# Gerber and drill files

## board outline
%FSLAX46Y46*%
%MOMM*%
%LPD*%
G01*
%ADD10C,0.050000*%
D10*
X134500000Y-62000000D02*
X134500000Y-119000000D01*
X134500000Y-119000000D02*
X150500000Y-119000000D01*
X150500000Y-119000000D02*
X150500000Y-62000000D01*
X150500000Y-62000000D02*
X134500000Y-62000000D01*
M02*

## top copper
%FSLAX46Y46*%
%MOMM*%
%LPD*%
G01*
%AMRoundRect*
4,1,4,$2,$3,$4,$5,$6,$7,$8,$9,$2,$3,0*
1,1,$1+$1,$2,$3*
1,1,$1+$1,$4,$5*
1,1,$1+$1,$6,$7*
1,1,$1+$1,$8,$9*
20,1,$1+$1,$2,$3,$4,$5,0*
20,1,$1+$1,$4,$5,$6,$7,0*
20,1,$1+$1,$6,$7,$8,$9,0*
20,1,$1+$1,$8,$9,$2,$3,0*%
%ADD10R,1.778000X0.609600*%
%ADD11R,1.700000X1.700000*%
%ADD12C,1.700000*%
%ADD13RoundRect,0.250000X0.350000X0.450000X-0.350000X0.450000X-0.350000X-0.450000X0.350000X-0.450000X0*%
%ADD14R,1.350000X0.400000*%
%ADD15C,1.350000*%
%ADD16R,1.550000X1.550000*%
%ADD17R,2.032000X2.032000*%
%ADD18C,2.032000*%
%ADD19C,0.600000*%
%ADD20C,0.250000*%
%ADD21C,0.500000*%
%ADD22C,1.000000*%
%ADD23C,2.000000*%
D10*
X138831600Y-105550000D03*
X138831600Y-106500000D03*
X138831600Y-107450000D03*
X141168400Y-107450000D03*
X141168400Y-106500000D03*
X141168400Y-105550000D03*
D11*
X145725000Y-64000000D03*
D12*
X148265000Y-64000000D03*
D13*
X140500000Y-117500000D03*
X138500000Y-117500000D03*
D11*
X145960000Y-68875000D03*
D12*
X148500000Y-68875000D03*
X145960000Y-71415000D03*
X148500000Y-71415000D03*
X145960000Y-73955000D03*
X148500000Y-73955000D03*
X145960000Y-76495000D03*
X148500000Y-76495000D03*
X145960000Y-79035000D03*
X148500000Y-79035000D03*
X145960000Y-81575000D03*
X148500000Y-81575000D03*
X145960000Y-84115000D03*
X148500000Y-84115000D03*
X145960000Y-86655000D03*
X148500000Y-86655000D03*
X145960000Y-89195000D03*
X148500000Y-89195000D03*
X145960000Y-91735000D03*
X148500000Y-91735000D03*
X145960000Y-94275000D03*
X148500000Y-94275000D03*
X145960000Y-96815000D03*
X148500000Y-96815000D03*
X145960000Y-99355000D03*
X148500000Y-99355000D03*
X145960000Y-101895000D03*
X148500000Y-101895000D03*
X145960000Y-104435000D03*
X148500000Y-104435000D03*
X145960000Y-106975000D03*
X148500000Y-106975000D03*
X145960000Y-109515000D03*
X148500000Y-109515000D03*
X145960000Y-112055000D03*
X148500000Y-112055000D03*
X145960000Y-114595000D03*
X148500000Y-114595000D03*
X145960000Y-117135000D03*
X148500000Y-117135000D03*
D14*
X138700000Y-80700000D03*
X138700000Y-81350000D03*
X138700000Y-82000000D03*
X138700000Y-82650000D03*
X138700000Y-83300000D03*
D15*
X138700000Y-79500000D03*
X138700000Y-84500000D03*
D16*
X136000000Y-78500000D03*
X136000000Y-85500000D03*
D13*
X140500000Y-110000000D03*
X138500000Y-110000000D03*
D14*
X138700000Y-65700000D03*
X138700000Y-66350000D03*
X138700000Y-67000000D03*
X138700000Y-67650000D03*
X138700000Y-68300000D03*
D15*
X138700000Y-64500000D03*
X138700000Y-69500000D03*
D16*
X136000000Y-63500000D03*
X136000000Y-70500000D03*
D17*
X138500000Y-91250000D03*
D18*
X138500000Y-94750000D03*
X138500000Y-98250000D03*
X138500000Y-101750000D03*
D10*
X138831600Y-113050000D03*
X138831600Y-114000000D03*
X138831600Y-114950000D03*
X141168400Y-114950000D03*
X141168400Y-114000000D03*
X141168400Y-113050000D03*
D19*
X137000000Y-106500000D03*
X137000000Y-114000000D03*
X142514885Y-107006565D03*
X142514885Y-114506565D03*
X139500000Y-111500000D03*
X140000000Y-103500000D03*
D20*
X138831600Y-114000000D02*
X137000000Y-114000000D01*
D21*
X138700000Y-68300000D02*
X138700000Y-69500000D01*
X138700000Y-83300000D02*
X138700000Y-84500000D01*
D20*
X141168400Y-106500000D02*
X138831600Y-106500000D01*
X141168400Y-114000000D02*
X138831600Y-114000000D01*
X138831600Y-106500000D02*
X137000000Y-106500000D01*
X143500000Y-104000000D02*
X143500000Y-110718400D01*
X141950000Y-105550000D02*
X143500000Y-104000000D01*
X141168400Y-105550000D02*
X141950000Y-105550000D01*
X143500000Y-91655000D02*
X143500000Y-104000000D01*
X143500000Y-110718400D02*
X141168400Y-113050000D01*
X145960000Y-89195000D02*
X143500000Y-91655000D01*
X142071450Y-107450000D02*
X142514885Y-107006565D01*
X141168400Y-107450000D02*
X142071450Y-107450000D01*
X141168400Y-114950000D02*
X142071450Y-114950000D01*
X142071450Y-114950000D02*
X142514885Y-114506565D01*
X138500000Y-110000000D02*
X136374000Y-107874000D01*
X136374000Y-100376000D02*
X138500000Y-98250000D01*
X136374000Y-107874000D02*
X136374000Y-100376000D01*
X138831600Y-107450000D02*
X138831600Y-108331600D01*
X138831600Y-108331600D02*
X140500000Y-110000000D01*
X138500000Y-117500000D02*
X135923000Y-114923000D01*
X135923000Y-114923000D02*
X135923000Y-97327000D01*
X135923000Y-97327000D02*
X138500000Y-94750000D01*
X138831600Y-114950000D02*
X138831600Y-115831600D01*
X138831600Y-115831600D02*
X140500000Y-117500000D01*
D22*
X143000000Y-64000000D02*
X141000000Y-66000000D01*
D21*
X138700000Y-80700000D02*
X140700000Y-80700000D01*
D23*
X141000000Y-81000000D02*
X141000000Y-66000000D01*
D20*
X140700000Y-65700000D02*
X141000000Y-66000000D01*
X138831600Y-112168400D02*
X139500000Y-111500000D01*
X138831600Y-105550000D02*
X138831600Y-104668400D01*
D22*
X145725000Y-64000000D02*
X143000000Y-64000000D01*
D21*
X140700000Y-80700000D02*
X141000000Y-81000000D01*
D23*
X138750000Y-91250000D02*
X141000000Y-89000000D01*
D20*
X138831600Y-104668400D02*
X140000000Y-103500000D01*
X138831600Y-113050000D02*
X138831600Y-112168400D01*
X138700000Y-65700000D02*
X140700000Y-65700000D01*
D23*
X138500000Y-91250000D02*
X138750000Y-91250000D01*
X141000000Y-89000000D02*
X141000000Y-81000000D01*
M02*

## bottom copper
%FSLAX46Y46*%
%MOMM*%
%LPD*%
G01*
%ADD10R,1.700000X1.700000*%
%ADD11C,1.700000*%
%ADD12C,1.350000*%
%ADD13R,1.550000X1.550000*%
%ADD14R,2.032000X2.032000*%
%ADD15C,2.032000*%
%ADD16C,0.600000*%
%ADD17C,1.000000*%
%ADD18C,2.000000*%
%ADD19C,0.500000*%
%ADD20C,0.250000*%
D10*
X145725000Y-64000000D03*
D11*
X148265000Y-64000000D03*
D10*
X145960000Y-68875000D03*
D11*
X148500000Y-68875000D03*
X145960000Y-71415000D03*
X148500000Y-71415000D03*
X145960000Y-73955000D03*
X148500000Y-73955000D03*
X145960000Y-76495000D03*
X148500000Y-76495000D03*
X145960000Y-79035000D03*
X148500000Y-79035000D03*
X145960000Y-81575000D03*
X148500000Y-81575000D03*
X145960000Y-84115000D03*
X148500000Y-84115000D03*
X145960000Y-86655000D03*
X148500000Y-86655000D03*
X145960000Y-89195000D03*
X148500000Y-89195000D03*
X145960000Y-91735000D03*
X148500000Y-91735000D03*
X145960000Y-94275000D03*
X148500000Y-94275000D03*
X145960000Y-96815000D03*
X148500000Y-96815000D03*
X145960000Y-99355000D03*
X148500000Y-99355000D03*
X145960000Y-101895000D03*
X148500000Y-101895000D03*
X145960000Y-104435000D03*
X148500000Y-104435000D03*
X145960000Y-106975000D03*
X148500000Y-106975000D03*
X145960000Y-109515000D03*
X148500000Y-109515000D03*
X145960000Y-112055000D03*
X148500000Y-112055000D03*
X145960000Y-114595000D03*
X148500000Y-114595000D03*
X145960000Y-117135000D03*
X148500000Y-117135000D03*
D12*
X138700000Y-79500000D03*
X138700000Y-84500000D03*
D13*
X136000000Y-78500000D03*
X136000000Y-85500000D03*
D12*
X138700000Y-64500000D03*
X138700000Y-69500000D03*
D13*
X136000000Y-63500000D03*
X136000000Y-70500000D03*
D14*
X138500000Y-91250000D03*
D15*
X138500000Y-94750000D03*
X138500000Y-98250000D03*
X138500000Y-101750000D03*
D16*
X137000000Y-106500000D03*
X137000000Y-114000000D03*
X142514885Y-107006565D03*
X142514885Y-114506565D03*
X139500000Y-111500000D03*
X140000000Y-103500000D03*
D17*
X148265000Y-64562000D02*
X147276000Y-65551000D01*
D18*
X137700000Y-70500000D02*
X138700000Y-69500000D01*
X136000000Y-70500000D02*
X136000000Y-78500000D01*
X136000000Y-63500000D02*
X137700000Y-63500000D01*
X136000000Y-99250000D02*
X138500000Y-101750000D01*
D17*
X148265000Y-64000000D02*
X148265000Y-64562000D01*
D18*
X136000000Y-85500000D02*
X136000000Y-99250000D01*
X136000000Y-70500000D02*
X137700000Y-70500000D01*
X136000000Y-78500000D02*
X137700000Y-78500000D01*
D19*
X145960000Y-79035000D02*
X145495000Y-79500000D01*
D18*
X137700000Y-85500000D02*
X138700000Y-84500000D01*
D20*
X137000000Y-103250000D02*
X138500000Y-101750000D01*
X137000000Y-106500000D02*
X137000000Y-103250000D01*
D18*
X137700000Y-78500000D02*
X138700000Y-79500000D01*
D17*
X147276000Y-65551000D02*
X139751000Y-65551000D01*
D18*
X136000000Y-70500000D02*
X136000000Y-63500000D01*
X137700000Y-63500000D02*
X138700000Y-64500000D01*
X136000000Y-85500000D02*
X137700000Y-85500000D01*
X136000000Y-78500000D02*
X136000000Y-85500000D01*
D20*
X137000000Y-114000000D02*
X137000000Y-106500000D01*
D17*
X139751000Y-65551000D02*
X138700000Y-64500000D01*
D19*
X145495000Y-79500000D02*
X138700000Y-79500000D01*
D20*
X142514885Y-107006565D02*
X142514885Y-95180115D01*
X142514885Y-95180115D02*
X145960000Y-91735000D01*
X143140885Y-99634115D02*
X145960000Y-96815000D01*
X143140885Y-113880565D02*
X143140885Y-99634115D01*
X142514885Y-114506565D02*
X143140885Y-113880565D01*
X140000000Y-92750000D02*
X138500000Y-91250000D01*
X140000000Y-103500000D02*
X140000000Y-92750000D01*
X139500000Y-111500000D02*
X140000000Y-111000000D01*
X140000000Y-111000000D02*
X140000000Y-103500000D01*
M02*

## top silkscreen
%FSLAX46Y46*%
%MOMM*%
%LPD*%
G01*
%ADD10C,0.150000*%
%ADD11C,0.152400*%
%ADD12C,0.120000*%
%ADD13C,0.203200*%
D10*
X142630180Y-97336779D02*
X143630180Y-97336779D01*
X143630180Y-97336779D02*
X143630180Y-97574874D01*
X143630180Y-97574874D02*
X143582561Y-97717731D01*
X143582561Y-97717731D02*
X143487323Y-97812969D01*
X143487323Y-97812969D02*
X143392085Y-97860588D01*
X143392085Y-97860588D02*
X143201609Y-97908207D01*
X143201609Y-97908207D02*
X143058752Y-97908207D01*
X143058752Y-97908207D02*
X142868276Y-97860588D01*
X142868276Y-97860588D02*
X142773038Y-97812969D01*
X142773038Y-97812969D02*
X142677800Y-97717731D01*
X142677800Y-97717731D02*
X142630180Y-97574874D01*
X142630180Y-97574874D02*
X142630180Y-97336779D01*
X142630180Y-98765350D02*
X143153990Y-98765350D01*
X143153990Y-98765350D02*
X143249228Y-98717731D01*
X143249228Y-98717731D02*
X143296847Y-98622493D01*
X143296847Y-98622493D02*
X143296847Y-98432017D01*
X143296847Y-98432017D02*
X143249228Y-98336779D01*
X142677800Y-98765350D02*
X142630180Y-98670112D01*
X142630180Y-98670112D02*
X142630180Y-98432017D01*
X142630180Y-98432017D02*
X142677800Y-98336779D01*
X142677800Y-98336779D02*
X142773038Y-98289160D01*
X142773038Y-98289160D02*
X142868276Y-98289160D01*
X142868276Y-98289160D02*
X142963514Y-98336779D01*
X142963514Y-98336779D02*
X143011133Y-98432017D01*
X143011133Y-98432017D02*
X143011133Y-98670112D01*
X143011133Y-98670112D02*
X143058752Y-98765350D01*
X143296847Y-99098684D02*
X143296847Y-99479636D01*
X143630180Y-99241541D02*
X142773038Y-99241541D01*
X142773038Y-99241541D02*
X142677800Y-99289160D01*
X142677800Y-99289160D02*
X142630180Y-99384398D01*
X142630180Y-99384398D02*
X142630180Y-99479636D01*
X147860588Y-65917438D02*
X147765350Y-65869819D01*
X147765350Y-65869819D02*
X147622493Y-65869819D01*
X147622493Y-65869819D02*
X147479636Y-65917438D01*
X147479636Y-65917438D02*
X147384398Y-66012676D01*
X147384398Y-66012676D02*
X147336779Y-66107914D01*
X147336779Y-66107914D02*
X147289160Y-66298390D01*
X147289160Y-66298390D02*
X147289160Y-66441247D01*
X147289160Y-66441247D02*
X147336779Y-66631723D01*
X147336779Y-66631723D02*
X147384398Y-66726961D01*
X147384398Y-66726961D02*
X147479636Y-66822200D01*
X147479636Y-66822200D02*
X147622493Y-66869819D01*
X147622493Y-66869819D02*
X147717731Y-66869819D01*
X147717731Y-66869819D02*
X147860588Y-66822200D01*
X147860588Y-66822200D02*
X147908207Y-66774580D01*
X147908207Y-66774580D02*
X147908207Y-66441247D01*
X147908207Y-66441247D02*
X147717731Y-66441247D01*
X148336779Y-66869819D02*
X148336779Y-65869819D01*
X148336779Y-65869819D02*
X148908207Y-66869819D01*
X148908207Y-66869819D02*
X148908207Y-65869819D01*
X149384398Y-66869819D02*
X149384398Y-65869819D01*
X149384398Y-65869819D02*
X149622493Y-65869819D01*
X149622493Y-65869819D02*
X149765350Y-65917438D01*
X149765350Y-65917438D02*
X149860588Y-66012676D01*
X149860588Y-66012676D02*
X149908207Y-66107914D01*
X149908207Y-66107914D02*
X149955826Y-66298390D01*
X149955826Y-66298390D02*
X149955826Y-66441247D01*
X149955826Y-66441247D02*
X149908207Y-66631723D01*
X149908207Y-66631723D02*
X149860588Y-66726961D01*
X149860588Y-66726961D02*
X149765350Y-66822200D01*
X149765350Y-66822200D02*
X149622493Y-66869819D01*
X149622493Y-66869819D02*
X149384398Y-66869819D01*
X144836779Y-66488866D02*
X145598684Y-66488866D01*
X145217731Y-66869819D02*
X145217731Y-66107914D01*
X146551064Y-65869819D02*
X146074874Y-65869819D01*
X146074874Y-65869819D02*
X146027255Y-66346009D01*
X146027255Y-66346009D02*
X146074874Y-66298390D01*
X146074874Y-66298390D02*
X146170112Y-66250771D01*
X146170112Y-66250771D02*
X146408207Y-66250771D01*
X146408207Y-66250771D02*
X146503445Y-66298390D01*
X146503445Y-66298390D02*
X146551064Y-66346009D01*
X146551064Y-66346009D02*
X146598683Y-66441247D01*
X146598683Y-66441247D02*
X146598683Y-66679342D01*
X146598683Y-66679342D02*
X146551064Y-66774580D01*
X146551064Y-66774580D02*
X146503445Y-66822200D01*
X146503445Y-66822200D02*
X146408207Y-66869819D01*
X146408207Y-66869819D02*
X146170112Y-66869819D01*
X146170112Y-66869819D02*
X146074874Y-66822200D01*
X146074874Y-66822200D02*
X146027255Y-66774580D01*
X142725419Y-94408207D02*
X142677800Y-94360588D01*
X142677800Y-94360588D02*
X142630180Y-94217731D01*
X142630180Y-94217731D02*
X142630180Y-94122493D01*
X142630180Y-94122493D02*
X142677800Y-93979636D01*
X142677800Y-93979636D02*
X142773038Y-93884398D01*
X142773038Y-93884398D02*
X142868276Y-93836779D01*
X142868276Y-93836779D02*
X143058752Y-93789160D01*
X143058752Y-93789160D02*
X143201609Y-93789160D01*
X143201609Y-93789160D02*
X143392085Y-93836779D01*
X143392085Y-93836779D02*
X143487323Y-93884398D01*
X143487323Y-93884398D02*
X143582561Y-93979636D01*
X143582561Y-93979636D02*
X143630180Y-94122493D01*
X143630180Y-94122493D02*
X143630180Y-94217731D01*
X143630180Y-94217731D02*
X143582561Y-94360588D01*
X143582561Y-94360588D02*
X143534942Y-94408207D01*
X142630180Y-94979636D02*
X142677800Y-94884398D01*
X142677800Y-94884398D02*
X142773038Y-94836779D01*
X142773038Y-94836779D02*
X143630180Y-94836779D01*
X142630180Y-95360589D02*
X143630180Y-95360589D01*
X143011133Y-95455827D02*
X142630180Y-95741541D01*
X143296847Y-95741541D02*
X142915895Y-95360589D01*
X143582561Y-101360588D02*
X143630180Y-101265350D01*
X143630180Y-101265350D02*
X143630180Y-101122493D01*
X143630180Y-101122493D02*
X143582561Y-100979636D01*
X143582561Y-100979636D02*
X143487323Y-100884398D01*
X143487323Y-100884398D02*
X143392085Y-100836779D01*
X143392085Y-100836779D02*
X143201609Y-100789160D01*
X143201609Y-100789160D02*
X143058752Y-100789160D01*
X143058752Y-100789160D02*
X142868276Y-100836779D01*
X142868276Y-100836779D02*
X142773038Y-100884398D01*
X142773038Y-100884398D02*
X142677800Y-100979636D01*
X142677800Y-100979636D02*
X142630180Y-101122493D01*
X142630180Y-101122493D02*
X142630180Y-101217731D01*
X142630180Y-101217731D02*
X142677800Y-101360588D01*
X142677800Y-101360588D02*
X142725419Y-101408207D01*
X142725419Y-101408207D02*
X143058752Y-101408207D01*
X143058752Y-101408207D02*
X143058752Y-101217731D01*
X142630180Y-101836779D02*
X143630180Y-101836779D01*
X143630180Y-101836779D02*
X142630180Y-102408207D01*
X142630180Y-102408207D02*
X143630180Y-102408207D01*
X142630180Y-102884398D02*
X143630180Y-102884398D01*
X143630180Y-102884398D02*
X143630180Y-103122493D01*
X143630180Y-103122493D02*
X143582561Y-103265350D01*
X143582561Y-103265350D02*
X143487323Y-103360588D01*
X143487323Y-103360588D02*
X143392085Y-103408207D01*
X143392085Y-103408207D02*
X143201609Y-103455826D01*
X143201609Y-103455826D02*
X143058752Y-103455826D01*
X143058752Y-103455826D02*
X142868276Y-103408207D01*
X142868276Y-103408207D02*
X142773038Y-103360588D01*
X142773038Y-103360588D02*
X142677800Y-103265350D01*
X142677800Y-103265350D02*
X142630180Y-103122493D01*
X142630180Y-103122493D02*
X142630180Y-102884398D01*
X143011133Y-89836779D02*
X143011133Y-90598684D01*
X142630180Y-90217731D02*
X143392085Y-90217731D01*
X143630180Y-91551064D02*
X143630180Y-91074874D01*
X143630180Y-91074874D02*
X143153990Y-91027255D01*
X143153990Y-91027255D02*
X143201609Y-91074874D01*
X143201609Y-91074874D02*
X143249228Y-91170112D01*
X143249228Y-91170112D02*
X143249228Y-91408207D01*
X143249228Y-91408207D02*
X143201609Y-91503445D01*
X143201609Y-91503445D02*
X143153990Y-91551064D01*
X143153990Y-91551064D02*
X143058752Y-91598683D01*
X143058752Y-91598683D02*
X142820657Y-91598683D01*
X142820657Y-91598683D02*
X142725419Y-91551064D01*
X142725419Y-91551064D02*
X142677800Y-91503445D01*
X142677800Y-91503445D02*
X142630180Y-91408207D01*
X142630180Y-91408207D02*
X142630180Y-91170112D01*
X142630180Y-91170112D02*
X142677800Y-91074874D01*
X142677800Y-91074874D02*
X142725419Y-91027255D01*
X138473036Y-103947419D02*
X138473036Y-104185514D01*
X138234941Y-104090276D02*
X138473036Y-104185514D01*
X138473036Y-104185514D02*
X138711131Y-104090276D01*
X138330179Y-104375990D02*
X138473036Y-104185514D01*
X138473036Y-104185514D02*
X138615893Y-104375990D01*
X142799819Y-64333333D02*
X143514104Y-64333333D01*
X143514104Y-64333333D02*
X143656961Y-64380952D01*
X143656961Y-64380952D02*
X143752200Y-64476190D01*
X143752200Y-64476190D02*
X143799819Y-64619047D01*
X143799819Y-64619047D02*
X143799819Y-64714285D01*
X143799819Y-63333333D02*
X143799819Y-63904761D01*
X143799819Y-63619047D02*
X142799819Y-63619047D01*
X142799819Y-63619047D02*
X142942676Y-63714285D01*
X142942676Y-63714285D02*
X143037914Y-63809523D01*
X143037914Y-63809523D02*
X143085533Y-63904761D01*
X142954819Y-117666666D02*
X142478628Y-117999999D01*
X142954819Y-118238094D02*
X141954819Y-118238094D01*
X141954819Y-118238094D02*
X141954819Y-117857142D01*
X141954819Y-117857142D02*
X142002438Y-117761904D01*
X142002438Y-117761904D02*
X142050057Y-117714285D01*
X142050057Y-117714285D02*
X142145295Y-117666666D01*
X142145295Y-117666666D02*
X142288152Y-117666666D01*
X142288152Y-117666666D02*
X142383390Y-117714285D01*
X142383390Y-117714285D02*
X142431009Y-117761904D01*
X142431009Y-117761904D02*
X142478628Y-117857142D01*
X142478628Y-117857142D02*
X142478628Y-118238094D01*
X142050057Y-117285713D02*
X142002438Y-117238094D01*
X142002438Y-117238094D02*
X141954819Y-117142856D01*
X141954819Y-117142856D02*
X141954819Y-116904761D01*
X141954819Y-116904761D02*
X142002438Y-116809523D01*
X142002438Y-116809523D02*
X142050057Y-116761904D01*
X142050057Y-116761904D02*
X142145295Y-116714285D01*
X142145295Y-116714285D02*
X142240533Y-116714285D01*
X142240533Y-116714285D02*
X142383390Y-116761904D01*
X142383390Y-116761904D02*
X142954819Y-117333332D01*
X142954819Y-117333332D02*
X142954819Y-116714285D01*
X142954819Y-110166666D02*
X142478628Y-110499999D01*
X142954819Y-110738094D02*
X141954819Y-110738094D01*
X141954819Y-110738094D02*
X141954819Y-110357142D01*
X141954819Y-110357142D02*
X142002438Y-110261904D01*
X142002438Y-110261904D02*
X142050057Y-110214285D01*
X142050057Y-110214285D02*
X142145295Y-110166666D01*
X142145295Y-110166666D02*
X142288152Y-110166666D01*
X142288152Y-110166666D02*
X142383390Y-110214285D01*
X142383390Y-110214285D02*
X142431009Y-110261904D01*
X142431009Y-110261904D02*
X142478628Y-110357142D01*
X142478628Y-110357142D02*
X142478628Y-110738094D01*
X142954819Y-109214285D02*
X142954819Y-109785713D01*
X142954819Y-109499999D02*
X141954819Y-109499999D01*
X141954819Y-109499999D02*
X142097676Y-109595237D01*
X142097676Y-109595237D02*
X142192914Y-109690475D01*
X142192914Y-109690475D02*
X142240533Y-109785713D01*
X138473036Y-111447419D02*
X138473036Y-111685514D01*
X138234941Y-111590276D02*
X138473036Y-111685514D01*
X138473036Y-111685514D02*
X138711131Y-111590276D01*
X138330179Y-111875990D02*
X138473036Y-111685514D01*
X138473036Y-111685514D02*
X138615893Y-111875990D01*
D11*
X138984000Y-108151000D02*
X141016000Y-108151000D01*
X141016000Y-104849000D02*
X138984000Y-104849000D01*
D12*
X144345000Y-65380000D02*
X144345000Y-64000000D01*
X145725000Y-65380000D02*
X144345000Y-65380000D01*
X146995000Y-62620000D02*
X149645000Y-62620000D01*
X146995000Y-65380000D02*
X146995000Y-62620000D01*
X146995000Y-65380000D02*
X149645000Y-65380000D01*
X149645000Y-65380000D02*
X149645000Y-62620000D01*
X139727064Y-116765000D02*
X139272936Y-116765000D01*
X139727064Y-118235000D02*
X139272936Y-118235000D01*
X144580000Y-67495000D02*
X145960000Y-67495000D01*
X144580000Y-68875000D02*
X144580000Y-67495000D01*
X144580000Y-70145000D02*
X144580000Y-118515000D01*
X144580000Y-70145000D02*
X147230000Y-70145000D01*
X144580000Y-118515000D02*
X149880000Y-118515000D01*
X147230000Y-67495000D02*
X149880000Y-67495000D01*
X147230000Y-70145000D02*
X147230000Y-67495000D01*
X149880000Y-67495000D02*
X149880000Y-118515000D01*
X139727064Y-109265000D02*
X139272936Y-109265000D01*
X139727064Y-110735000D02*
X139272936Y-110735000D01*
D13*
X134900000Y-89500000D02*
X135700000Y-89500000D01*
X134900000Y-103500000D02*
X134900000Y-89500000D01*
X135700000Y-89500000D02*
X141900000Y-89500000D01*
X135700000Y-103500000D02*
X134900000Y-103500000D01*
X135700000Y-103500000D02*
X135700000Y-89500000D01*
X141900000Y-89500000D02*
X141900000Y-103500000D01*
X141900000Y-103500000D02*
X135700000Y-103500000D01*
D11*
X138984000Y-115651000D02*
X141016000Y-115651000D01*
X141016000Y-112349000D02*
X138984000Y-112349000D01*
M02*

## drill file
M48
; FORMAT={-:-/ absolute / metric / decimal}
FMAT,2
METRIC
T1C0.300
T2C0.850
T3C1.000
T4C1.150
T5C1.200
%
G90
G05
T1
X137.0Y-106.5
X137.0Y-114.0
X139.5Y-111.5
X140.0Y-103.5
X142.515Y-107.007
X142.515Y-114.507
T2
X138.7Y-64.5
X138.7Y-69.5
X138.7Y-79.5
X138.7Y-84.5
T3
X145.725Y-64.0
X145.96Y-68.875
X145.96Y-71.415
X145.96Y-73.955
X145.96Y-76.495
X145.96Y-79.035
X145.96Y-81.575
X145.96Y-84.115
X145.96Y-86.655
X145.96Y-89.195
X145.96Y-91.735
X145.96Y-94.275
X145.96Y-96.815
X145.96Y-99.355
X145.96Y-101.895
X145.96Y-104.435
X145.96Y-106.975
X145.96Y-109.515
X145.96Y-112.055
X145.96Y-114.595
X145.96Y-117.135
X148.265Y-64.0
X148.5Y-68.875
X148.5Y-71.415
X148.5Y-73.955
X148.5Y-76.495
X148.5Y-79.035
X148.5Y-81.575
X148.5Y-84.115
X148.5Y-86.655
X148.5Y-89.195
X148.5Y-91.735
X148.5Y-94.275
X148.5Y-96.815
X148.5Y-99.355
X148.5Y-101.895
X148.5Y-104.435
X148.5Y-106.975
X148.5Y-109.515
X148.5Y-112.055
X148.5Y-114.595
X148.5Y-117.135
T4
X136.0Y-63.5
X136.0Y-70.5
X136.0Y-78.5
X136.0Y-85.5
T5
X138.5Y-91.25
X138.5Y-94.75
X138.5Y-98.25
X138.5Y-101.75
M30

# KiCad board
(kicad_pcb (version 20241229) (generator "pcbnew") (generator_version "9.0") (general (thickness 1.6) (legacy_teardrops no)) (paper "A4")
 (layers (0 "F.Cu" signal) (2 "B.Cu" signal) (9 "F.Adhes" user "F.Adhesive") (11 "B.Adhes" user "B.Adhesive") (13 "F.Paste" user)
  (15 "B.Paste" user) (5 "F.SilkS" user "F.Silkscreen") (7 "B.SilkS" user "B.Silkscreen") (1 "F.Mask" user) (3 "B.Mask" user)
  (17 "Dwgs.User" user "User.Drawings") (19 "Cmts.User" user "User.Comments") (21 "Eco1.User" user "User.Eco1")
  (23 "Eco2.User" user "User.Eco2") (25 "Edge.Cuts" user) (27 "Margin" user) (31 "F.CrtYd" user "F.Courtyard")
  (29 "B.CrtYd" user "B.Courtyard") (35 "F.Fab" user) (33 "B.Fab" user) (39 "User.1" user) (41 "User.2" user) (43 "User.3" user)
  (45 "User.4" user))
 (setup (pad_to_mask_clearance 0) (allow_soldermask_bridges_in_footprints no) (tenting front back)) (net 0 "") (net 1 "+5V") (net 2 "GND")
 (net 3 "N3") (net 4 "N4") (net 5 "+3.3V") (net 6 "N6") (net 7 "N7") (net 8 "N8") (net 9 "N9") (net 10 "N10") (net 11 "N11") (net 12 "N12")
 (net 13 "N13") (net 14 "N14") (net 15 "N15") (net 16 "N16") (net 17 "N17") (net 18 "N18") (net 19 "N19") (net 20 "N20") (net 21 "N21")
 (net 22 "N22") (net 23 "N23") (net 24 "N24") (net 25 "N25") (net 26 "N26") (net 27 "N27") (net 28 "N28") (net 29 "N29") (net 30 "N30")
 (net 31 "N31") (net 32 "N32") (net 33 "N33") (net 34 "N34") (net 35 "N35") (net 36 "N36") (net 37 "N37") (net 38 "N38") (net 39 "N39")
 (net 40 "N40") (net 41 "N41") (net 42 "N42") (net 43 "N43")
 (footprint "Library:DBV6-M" (layer "F.Cu") (at 140 106.5)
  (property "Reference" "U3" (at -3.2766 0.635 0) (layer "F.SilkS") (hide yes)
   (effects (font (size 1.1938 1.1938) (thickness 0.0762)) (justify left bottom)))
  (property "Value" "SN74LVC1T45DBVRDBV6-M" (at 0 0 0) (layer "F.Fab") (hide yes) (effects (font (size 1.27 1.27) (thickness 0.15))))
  (fp_line (start -1.016 1.651) (end 1.016 1.651) (stroke (width 0.1524) (type solid)) (layer "F.SilkS"))
  (fp_line (start 1.016 -1.651) (end -1.016 -1.651) (stroke (width 0.1524) (type solid)) (layer "F.SilkS"))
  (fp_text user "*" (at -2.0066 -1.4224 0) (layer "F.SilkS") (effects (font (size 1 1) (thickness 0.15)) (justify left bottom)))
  (pad "1" smd rect (at -1.1684 -0.95) (size 1.778 0.6096) (layers "F.Cu" "F.Mask" "F.Paste") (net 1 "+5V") (solder_mask_margin 0.0635)
   (thermal_bridge_angle 0))
  (pad "2" smd rect (at -1.1684 0) (size 1.778 0.6096) (layers "F.Cu" "F.Mask" "F.Paste") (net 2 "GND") (solder_mask_margin 0.0635)
   (thermal_bridge_angle 0))
  (pad "3" smd rect (at -1.1684 0.95) (size 1.778 0.6096) (layers "F.Cu" "F.Mask" "F.Paste") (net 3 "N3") (solder_mask_margin 0.0635)
   (thermal_bridge_angle 0))
  (pad "4" smd rect (at 1.1684 0.95) (size 1.778 0.6096) (layers "F.Cu" "F.Mask" "F.Paste") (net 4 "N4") (solder_mask_margin 0.0635)
   (thermal_bridge_angle 0))
  (pad "5" smd rect (at 1.1684 0) (size 1.778 0.6096) (layers "F.Cu" "F.Mask" "F.Paste") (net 2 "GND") (solder_mask_margin 0.0635)
   (thermal_bridge_angle 0))
  (pad "6" smd rect (at 1.1684 -0.95) (size 1.778 0.6096) (layers "F.Cu" "F.Mask" "F.Paste") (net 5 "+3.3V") (solder_mask_margin 0.0635)
   (thermal_bridge_angle 0)))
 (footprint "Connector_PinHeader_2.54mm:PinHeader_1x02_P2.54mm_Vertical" (layer "F.Cu") (at 145.725 64 90)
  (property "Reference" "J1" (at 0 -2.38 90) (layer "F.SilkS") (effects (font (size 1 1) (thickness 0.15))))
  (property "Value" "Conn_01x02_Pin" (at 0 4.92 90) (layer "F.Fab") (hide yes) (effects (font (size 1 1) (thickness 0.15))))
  (fp_line (start -1.38 -1.38) (end 0 -1.38) (stroke (width 0.12) (type solid)) (layer "F.SilkS"))
  (fp_line (start -1.38 0) (end -1.38 -1.38) (stroke (width 0.12) (type solid)) (layer "F.SilkS"))
  (fp_line (start 1.38 1.27) (end 1.38 3.92) (stroke (width 0.12) (type solid)) (layer "F.SilkS"))
  (fp_line (start -1.38 1.27) (end 1.38 1.27) (stroke (width 0.12) (type solid)) (layer "F.SilkS"))
  (fp_line (start -1.38 1.27) (end -1.38 3.92) (stroke (width 0.12) (type solid)) (layer "F.SilkS"))
  (fp_line (start -1.38 3.92) (end 1.38 3.92) (stroke (width 0.12) (type solid)) (layer "F.SilkS"))
  (pad "1" thru_hole rect (at 0 0 90) (size 1.7 1.7) (drill 1) (layers "*.Cu" "*.Mask") (remove_unused_layers no) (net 1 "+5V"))
  (pad "2" thru_hole circle (at 0 2.54 90) (size 1.7 1.7) (drill 1) (layers "*.Cu" "*.Mask") (remove_unused_layers no) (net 2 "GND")))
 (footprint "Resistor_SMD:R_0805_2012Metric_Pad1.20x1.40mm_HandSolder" (layer "F.Cu") (at 139.5 117.5 180)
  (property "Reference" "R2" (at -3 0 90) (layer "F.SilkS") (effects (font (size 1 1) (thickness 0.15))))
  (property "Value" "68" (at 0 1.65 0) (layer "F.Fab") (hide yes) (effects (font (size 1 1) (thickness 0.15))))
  (fp_line (start -0.227064 0.735) (end 0.227064 0.735) (stroke (width 0.12) (type solid)) (layer "F.SilkS"))
  (fp_line (start -0.227064 -0.735) (end 0.227064 -0.735) (stroke (width 0.12) (type solid)) (layer "F.SilkS"))
  (pad "1" smd roundrect (at -1 0 180) (size 1.2 1.4) (layers "F.Cu" "F.Mask" "F.Paste") (roundrect_rratio 0.208333) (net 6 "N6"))
  (pad "2" smd roundrect (at 1 0 180) (size 1.2 1.4) (layers "F.Cu" "F.Mask" "F.Paste") (roundrect_rratio 0.208333) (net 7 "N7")))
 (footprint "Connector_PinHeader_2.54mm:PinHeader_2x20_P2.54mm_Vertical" (layer "F.Cu") (at 145.96 68.875)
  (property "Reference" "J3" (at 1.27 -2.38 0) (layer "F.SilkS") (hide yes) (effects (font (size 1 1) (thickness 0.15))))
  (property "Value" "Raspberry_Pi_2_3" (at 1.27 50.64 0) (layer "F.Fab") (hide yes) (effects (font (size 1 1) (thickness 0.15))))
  (fp_line (start -1.38 -1.38) (end 0 -1.38) (stroke (width 0.12) (type solid)) (layer "F.SilkS"))
  (fp_line (start -1.38 0) (end -1.38 -1.38) (stroke (width 0.12) (type solid)) (layer "F.SilkS"))
  (fp_line (start -1.38 1.27) (end -1.38 49.64) (stroke (width 0.12) (type solid)) (layer "F.SilkS"))
  (fp_line (start -1.38 1.27) (end 1.27 1.27) (stroke (width 0.12) (type solid)) (layer "F.SilkS"))
  (fp_line (start -1.38 49.64) (end 3.92 49.64) (stroke (width 0.12) (type solid)) (layer "F.SilkS"))
  (fp_line (start 1.27 -1.38) (end 3.92 -1.38) (stroke (width 0.12) (type solid)) (layer "F.SilkS"))
  (fp_line (start 1.27 1.27) (end 1.27 -1.38) (stroke (width 0.12) (type solid)) (layer "F.SilkS"))
  (fp_line (start 3.92 -1.38) (end 3.92 49.64) (stroke (width 0.12) (type solid)) (layer "F.SilkS"))
  (pad "1" thru_hole rect (at 0 0) (size 1.7 1.7) (drill 1) (layers "*.Cu" "*.Mask") (remove_unused_layers no) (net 5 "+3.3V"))
  (pad "2" thru_hole circle (at 2.54 0) (size 1.7 1.7) (drill 1) (layers "*.Cu" "*.Mask") (remove_unused_layers no) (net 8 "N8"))
  (pad "3" thru_hole circle (at 0 2.54) (size 1.7 1.7) (drill 1) (layers "*.Cu" "*.Mask") (remove_unused_layers no) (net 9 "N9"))
  (pad "4" thru_hole circle (at 2.54 2.54) (size 1.7 1.7) (drill 1) (layers "*.Cu" "*.Mask") (remove_unused_layers no) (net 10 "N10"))
  (pad "5" thru_hole circle (at 0 5.08) (size 1.7 1.7) (drill 1) (layers "*.Cu" "*.Mask") (remove_unused_layers no) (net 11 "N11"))
  (pad "6" thru_hole circle (at 2.54 5.08) (size 1.7 1.7) (drill 1) (layers "*.Cu" "*.Mask") (remove_unused_layers no) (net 2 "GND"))
  (pad "7" thru_hole circle (at 0 7.62) (size 1.7 1.7) (drill 1) (layers "*.Cu" "*.Mask") (remove_unused_layers no) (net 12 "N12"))
  (pad "8" thru_hole circle (at 2.54 7.62) (size 1.7 1.7) (drill 1) (layers "*.Cu" "*.Mask") (remove_unused_layers no) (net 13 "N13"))
  (pad "9" thru_hole circle (at 0 10.16) (size 1.7 1.7) (drill 1) (layers "*.Cu" "*.Mask") (remove_unused_layers no) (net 2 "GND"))
  (pad "10" thru_hole circle (at 2.54 10.16) (size 1.7 1.7) (drill 1) (layers "*.Cu" "*.Mask") (remove_unused_layers no) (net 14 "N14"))
  (pad "11" thru_hole circle (at 0 12.7) (size 1.7 1.7) (drill 1) (layers "*.Cu" "*.Mask") (remove_unused_layers no) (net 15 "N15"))
  (pad "12" thru_hole circle (at 2.54 12.7) (size 1.7 1.7) (drill 1) (layers "*.Cu" "*.Mask") (remove_unused_layers no) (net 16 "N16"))
  (pad "13" thru_hole circle (at 0 15.24) (size 1.7 1.7) (drill 1) (layers "*.Cu" "*.Mask") (remove_unused_layers no) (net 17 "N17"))
  (pad "14" thru_hole circle (at 2.54 15.24) (size 1.7 1.7) (drill 1) (layers "*.Cu" "*.Mask") (remove_unused_layers no) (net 2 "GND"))
  (pad "15" thru_hole circle (at 0 17.78) (size 1.7 1.7) (drill 1) (layers "*.Cu" "*.Mask") (remove_unused_layers no) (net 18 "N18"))
  (pad "16" thru_hole circle (at 2.54 17.78) (size 1.7 1.7) (drill 1) (layers "*.Cu" "*.Mask") (remove_unused_layers no) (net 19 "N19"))
  (pad "17" thru_hole circle (at 0 20.32) (size 1.7 1.7) (drill 1) (layers "*.Cu" "*.Mask") (remove_unused_layers no) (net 5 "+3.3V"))
  (pad "18" thru_hole circle (at 2.54 20.32) (size 1.7 1.7) (drill 1) (layers "*.Cu" "*.Mask") (remove_unused_layers no) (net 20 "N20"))
  (pad "19" thru_hole circle (at 0 22.86) (size 1.7 1.7) (drill 1) (layers "*.Cu" "*.Mask") (remove_unused_layers no) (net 4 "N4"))
  (pad "20" thru_hole circle (at 2.54 22.86) (size 1.7 1.7) (drill 1) (layers "*.Cu" "*.Mask") (remove_unused_layers no) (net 2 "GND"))
  (pad "21" thru_hole circle (at 0 25.4) (size 1.7 1.7) (drill 1) (layers "*.Cu" "*.Mask") (remove_unused_layers no) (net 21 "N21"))
  (pad "22" thru_hole circle (at 2.54 25.4) (size 1.7 1.7) (drill 1) (layers "*.Cu" "*.Mask") (remove_unused_layers no) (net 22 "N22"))
  (pad "23" thru_hole circle (at 0 27.94) (size 1.7 1.7) (drill 1) (layers "*.Cu" "*.Mask") (remove_unused_layers no) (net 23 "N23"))
  (pad "24" thru_hole circle (at 2.54 27.94) (size 1.7 1.7) (drill 1) (layers "*.Cu" "*.Mask") (remove_unused_layers no) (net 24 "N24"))
  (pad "25" thru_hole circle (at 0 30.48) (size 1.7 1.7) (drill 1) (layers "*.Cu" "*.Mask") (remove_unused_layers no) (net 2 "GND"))
  (pad "26" thru_hole circle (at 2.54 30.48) (size 1.7 1.7) (drill 1) (layers "*.Cu" "*.Mask") (remove_unused_layers no) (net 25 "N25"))
  (pad "27" thru_hole circle (at 0 33.02) (size 1.7 1.7) (drill 1) (layers "*.Cu" "*.Mask") (remove_unused_layers no) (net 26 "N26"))
  (pad "28" thru_hole circle (at 2.54 33.02) (size 1.7 1.7) (drill 1) (layers "*.Cu" "*.Mask") (remove_unused_layers no) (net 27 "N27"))
  (pad "29" thru_hole circle (at 0 35.56) (size 1.7 1.7) (drill 1) (layers "*.Cu" "*.Mask") (remove_unused_layers no) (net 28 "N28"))
  (pad "30" thru_hole circle (at 2.54 35.56) (size 1.7 1.7) (drill 1) (layers "*.Cu" "*.Mask") (remove_unused_layers no) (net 2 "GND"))
  (pad "31" thru_hole circle (at 0 38.1) (size 1.7 1.7) (drill 1) (layers "*.Cu" "*.Mask") (remove_unused_layers no) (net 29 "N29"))
  (pad "32" thru_hole circle (at 2.54 38.1) (size 1.7 1.7) (drill 1) (layers "*.Cu" "*.Mask") (remove_unused_layers no) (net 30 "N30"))
  (pad "33" thru_hole circle (at 0 40.64) (size 1.7 1.7) (drill 1) (layers "*.Cu" "*.Mask") (remove_unused_layers no) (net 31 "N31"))
  (pad "34" thru_hole circle (at 2.54 40.64) (size 1.7 1.7) (drill 1) (layers "*.Cu" "*.Mask") (remove_unused_layers no) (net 2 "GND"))
  (pad "35" thru_hole circle (at 0 43.18) (size 1.7 1.7) (drill 1) (layers "*.Cu" "*.Mask") (remove_unused_layers no) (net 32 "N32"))
  (pad "36" thru_hole circle (at 2.54 43.18) (size 1.7 1.7) (drill 1) (layers "*.Cu" "*.Mask") (remove_unused_layers no) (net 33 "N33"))
  (pad "37" thru_hole circle (at 0 45.72) (size 1.7 1.7) (drill 1) (layers "*.Cu" "*.Mask") (remove_unused_layers no) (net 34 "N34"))
  (pad "38" thru_hole circle (at 2.54 45.72) (size 1.7 1.7) (drill 1) (layers "*.Cu" "*.Mask") (remove_unused_layers no) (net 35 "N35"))
  (pad "39" thru_hole circle (at 0 48.26) (size 1.7 1.7) (drill 1) (layers "*.Cu" "*.Mask") (remove_unused_layers no) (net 2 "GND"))
  (pad "40" thru_hole circle (at 2.54 48.26) (size 1.7 1.7) (drill 1) (layers "*.Cu" "*.Mask") (remove_unused_layers no) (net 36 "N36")))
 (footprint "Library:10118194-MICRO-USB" (layer "F.Cu") (at 136 82 -90)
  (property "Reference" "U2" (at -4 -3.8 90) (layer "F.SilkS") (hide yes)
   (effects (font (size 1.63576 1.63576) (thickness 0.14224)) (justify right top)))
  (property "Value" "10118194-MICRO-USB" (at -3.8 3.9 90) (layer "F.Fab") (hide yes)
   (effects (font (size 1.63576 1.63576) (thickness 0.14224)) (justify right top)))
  (pad "1" smd rect (at -1.3 -2.7 90) (size 0.4 1.35) (layers "F.Cu" "F.Mask" "F.Paste") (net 1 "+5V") (solder_mask_margin 0.0635)
   (thermal_bridge_angle 0))
  (pad "2" smd rect (at -0.65 -2.7 90) (size 0.4 1.35) (layers "F.Cu" "F.Mask" "F.Paste") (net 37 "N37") (solder_mask_margin 0.0635)
   (thermal_bridge_angle 0))
  (pad "3" smd rect (at 0 -2.7 90) (size 0.4 1.35) (layers "F.Cu" "F.Mask" "F.Paste") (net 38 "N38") (solder_mask_margin 0.0635)
   (thermal_bridge_angle 0))
  (pad "4" smd rect (at 0.65 -2.7 90) (size 0.4 1.35) (layers "F.Cu" "F.Mask" "F.Paste") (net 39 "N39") (solder_mask_margin 0.0635)
   (thermal_bridge_angle 0))
  (pad "5" smd rect (at 1.3 -2.7 90) (size 0.4 1.35) (layers "F.Cu" "F.Mask" "F.Paste") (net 2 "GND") (solder_mask_margin 0.0635)
   (thermal_bridge_angle 0))
  (pad "M1" thru_hole circle (at -2.5 -2.7 270) (size 1.35 1.35) (drill 0.85) (layers "*.Cu" "*.Mask") (remove_unused_layers no)
   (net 2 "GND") (solder_mask_margin 0.0635) (thermal_bridge_angle 0))
  (pad "M2" thru_hole circle (at 2.5 -2.7 270) (size 1.35 1.35) (drill 0.85) (layers "*.Cu" "*.Mask") (remove_unused_layers no)
   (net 2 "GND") (solder_mask_margin 0.0635) (thermal_bridge_angle 0))
  (pad "M3" thru_hole rect (at -3.5 0 270) (size 1.55 1.55) (drill 1.15) (layers "*.Cu" "*.Mask") (remove_unused_layers no) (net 2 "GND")
   (solder_mask_margin 0.0635) (thermal_bridge_angle 0))
  (pad "M4" thru_hole rect (at 3.5 0 270) (size 1.55 1.55) (drill 1.15) (layers "*.Cu" "*.Mask") (remove_unused_layers no) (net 2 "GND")
   (solder_mask_margin 0.0635) (thermal_bridge_angle 0)))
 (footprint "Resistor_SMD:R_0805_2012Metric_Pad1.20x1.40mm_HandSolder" (layer "F.Cu") (at 139.5 110 180)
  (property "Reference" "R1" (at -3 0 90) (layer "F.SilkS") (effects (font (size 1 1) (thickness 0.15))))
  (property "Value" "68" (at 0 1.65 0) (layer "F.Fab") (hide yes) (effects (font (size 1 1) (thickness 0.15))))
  (fp_line (start -0.227064 0.735) (end 0.227064 0.735) (stroke (width 0.12) (type solid)) (layer "F.SilkS"))
  (fp_line (start -0.227064 -0.735) (end 0.227064 -0.735) (stroke (width 0.12) (type solid)) (layer "F.SilkS"))
  (pad "1" smd roundrect (at -1 0 180) (size 1.2 1.4) (layers "F.Cu" "F.Mask" "F.Paste") (roundrect_rratio 0.208333) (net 3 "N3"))
  (pad "2" smd roundrect (at 1 0 180) (size 1.2 1.4) (layers "F.Cu" "F.Mask" "F.Paste") (roundrect_rratio 0.208333) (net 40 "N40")))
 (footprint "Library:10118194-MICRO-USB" (layer "F.Cu") (at 136 67 -90)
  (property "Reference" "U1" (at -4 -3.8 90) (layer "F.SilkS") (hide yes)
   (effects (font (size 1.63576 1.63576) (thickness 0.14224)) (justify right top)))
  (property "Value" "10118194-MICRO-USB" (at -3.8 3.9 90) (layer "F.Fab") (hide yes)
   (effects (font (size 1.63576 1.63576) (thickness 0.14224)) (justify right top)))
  (pad "1" smd rect (at -1.3 -2.7 90) (size 0.4 1.35) (layers "F.Cu" "F.Mask" "F.Paste") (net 1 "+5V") (solder_mask_margin 0.0635)
   (thermal_bridge_angle 0))
  (pad "2" smd rect (at -0.65 -2.7 90) (size 0.4 1.35) (layers "F.Cu" "F.Mask" "F.Paste") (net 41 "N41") (solder_mask_margin 0.0635)
   (thermal_bridge_angle 0))
  (pad "3" smd rect (at 0 -2.7 90) (size 0.4 1.35) (layers "F.Cu" "F.Mask" "F.Paste") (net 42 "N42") (solder_mask_margin 0.0635)
   (thermal_bridge_angle 0))
  (pad "4" smd rect (at 0.65 -2.7 90) (size 0.4 1.35) (layers "F.Cu" "F.Mask" "F.Paste") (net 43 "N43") (solder_mask_margin 0.0635)
   (thermal_bridge_angle 0))
  (pad "5" smd rect (at 1.3 -2.7 90) (size 0.4 1.35) (layers "F.Cu" "F.Mask" "F.Paste") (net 2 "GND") (solder_mask_margin 0.0635)
   (thermal_bridge_angle 0))
  (pad "M1" thru_hole circle (at -2.5 -2.7 270) (size 1.35 1.35) (drill 0.85) (layers "*.Cu" "*.Mask") (remove_unused_layers no)
   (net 2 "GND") (solder_mask_margin 0.0635) (thermal_bridge_angle 0))
  (pad "M2" thru_hole circle (at 2.5 -2.7 270) (size 1.35 1.35) (drill 0.85) (layers "*.Cu" "*.Mask") (remove_unused_layers no)
   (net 2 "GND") (solder_mask_margin 0.0635) (thermal_bridge_angle 0))
  (pad "M3" thru_hole rect (at -3.5 0 270) (size 1.55 1.55) (drill 1.15) (layers "*.Cu" "*.Mask") (remove_unused_layers no) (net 2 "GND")
   (solder_mask_margin 0.0635) (thermal_bridge_angle 0))
  (pad "M4" thru_hole rect (at 3.5 0 270) (size 1.55 1.55) (drill 1.15) (layers "*.Cu" "*.Mask") (remove_unused_layers no) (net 2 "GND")
   (solder_mask_margin 0.0635) (thermal_bridge_angle 0)))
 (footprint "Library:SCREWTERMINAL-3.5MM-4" (layer "F.Cu") (at 138.5 91.25 -90)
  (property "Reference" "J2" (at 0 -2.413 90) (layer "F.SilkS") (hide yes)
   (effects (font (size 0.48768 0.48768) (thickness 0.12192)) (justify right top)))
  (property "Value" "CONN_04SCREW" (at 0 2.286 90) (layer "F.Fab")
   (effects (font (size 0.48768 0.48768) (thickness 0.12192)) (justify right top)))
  (fp_line (start -1.75 3.6) (end -1.75 2.8) (stroke (width 0.2032) (type solid)) (layer "F.SilkS"))
  (fp_line (start 12.25 3.6) (end -1.75 3.6) (stroke (width 0.2032) (type solid)) (layer "F.SilkS"))
  (fp_line (start -1.75 2.8) (end -1.75 -3.4) (stroke (width 0.2032) (type solid)) (layer "F.SilkS"))
  (fp_line (start 12.25 2.8) (end 12.25 3.6) (stroke (width 0.2032) (type solid)) (layer "F.SilkS"))
  (fp_line (start 12.25 2.8) (end -1.75 2.8) (stroke (width 0.2032) (type solid)) (layer "F.SilkS"))
  (fp_line (start -1.75 -3.4) (end 12.25 -3.4) (stroke (width 0.2032) (type solid)) (layer "F.SilkS"))
  (fp_line (start 12.25 -3.4) (end 12.25 2.8) (stroke (width 0.2032) (type solid)) (layer "F.SilkS"))
  (pad "1" thru_hole rect (at 0 0 270) (size 2.032 2.032) (drill 1.2) (layers "*.Cu" "*.Mask") (remove_unused_layers no) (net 1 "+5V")
   (solder_mask_margin 0.0635) (thermal_bridge_angle 0))
  (pad "2" thru_hole circle (at 3.5 0 270) (size 2.032 2.032) (drill 1.2) (layers "*.Cu" "*.Mask") (remove_unused_layers no) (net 7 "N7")
   (solder_mask_margin 0.0635) (thermal_bridge_angle 0))
  (pad "3" thru_hole circle (at 7 0 270) (size 2.032 2.032) (drill 1.2) (layers "*.Cu" "*.Mask") (remove_unused_layers no) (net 40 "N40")
   (solder_mask_margin 0.0635) (thermal_bridge_angle 0))
  (pad "4" thru_hole circle (at 10.5 0 270) (size 2.032 2.032) (drill 1.2) (layers "*.Cu" "*.Mask") (remove_unused_layers no) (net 2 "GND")
   (solder_mask_margin 0.0635) (thermal_bridge_angle 0)))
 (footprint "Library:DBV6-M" (layer "F.Cu") (at 140 114)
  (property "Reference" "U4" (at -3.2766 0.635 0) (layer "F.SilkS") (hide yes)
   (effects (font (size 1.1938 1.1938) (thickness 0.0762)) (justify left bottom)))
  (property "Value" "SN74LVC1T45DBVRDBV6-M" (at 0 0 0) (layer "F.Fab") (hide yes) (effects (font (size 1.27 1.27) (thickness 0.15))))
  (fp_line (start -1.016 1.651) (end 1.016 1.651) (stroke (width 0.1524) (type solid)) (layer "F.SilkS"))
  (fp_line (start 1.016 -1.651) (end -1.016 -1.651) (stroke (width 0.1524) (type solid)) (layer "F.SilkS"))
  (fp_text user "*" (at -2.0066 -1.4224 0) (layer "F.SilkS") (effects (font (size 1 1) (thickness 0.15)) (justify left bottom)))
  (pad "1" smd rect (at -1.1684 -0.95) (size 1.778 0.6096) (layers "F.Cu" "F.Mask" "F.Paste") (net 1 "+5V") (solder_mask_margin 0.0635)
   (thermal_bridge_angle 0))
  (pad "2" smd rect (at -1.1684 0) (size 1.778 0.6096) (layers "F.Cu" "F.Mask" "F.Paste") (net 2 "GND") (solder_mask_margin 0.0635)
   (thermal_bridge_angle 0))
  (pad "3" smd rect (at -1.1684 0.95) (size 1.778 0.6096) (layers "F.Cu" "F.Mask" "F.Paste") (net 6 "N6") (solder_mask_margin 0.0635)
   (thermal_bridge_angle 0))
  (pad "4" smd rect (at 1.1684 0.95) (size 1.778 0.6096) (layers "F.Cu" "F.Mask" "F.Paste") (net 23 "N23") (solder_mask_margin 0.0635)
   (thermal_bridge_angle 0))
  (pad "5" smd rect (at 1.1684 0) (size 1.778 0.6096) (layers "F.Cu" "F.Mask" "F.Paste") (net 2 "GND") (solder_mask_margin 0.0635)
   (thermal_bridge_angle 0))
  (pad "6" smd rect (at 1.1684 -0.95) (size 1.778 0.6096) (layers "F.Cu" "F.Mask" "F.Paste") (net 5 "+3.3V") (solder_mask_margin 0.0635)
   (thermal_bridge_angle 0)))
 (gr_line (start 134.5 62) (end 134.5 119) (stroke (width 0.05) (type default)) (layer "Edge.Cuts"))
 (gr_line (start 134.5 119) (end 150.5 119) (stroke (width 0.05) (type default)) (layer "Edge.Cuts"))
 (gr_line (start 150.5 119) (end 150.5 62) (stroke (width 0.05) (type default)) (layer "Edge.Cuts"))
 (gr_line (start 150.5 62) (end 134.5 62) (stroke (width 0.05) (type default)) (layer "Edge.Cuts"))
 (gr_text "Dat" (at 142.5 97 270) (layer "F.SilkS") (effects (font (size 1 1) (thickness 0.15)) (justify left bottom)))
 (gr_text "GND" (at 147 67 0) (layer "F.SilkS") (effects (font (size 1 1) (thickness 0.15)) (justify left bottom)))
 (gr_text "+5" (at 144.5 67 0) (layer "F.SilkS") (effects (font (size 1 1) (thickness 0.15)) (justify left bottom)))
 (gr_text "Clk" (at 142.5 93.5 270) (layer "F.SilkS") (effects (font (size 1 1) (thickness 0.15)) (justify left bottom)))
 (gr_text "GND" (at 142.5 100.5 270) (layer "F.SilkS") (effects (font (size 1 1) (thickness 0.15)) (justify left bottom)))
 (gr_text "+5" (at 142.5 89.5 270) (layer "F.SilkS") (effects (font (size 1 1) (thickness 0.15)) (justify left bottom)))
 (segment (start 138.8316 114) (end 137 114) (width 0.25) (layer "F.Cu") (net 2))
 (segment (start 138.7 68.3) (end 138.7 69.5) (width 0.5) (layer "F.Cu") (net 2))
 (segment (start 138.7 83.3) (end 138.7 84.5) (width 0.5) (layer "F.Cu") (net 2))
 (segment (start 141.1684 106.5) (end 138.8316 106.5) (width 0.25) (layer "F.Cu") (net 2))
 (segment (start 141.1684 114) (end 138.8316 114) (width 0.25) (layer "F.Cu") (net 2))
 (segment (start 138.8316 106.5) (end 137 106.5) (width 0.25) (layer "F.Cu") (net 2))
 (via (at 137 106.5) (size 0.6) (drill 0.3) (layers "F.Cu" "B.Cu") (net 2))
 (via (at 137 114) (size 0.6) (drill 0.3) (layers "F.Cu" "B.Cu") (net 2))
 (segment (start 148.265 64.562) (end 147.276 65.551) (width 1) (layer "B.Cu") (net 2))
 (segment (start 137.7 70.5) (end 138.7 69.5) (width 2) (layer "B.Cu") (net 2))
 (segment (start 136 70.5) (end 136 78.5) (width 2) (layer "B.Cu") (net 2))
 (segment (start 136 63.5) (end 137.7 63.5) (width 2) (layer "B.Cu") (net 2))
 (segment (start 136 99.25) (end 138.5 101.75) (width 2) (layer "B.Cu") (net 2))
 (segment (start 148.265 64) (end 148.265 64.562) (width 1) (layer "B.Cu") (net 2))
 (segment (start 136 85.5) (end 136 99.25) (width 2) (layer "B.Cu") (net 2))
 (segment (start 136 70.5) (end 137.7 70.5) (width 2) (layer "B.Cu") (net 2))
 (segment (start 136 78.5) (end 137.7 78.5) (width 2) (layer "B.Cu") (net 2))
 (segment (start 145.96 79.035) (end 145.495 79.5) (width 0.5) (layer "B.Cu") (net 2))
 (segment (start 137.7 85.5) (end 138.7 84.5) (width 2) (layer "B.Cu") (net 2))
 (segment (start 137 103.25) (end 138.5 101.75) (width 0.25) (layer "B.Cu") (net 2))
 (segment (start 137 106.5) (end 137 103.25) (width 0.25) (layer "B.Cu") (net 2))
 (segment (start 137.7 78.5) (end 138.7 79.5) (width 2) (layer "B.Cu") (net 2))
 (segment (start 147.276 65.551) (end 139.751 65.551) (width 1) (layer "B.Cu") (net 2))
 (segment (start 136 70.5) (end 136 63.5) (width 2) (layer "B.Cu") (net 2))
 (segment (start 137.7 63.5) (end 138.7 64.5) (width 2) (layer "B.Cu") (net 2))
 (segment (start 136 85.5) (end 137.7 85.5) (width 2) (layer "B.Cu") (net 2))
 (segment (start 136 78.5) (end 136 85.5) (width 2) (layer "B.Cu") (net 2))
 (segment (start 137 114) (end 137 106.5) (width 0.25) (layer "B.Cu") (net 2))
 (segment (start 139.751 65.551) (end 138.7 64.5) (width 1) (layer "B.Cu") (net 2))
 (segment (start 145.495 79.5) (end 138.7 79.5) (width 0.5) (layer "B.Cu") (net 2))
 (segment (start 143.5 104) (end 143.5 110.7184) (width 0.25) (layer "F.Cu") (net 5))
 (segment (start 141.95 105.55) (end 143.5 104) (width 0.25) (layer "F.Cu") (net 5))
 (segment (start 141.1684 105.55) (end 141.95 105.55) (width 0.25) (layer "F.Cu") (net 5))
 (segment (start 143.5 91.655) (end 143.5 104) (width 0.25) (layer "F.Cu") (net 5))
 (segment (start 143.5 110.7184) (end 141.1684 113.05) (width 0.25) (layer "F.Cu") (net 5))
 (segment (start 145.96 89.195) (end 143.5 91.655) (width 0.25) (layer "F.Cu") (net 5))
 (segment (start 142.07145 107.45) (end 142.514885 107.006565) (width 0.25) (layer "F.Cu") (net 4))
 (segment (start 141.1684 107.45) (end 142.07145 107.45) (width 0.25) (layer "F.Cu") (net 4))
 (via (at 142.514885 107.006565) (size 0.6) (drill 0.3) (layers "F.Cu" "B.Cu") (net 4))
 (segment (start 142.514885 107.006565) (end 142.514885 95.180115) (width 0.25) (layer "B.Cu") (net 4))
 (segment (start 142.514885 95.180115) (end 145.96 91.735) (width 0.25) (layer "B.Cu") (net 4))
 (segment (start 141.1684 114.95) (end 142.07145 114.95) (width 0.25) (layer "F.Cu") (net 23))
 (segment (start 142.07145 114.95) (end 142.514885 114.506565) (width 0.25) (layer "F.Cu") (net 23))
 (via (at 142.514885 114.506565) (size 0.6) (drill 0.3) (layers "F.Cu" "B.Cu") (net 23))
 (segment (start 143.140885 99.634115) (end 145.96 96.815) (width 0.25) (layer "B.Cu") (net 23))
 (segment (start 143.140885 113.880565) (end 143.140885 99.634115) (width 0.25) (layer "B.Cu") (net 23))
 (segment (start 142.514885 114.506565) (end 143.140885 113.880565) (width 0.25) (layer "B.Cu") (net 23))
 (segment (start 138.5 110) (end 136.374 107.874) (width 0.25) (layer "F.Cu") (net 40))
 (segment (start 136.374 100.376) (end 138.5 98.25) (width 0.25) (layer "F.Cu") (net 40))
 (segment (start 136.374 107.874) (end 136.374 100.376) (width 0.25) (layer "F.Cu") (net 40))
 (segment (start 138.8316 107.45) (end 138.8316 108.3316) (width 0.25) (layer "F.Cu") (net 3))
 (segment (start 138.8316 108.3316) (end 140.5 110) (width 0.25) (layer "F.Cu") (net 3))
 (segment (start 138.5 117.5) (end 135.923 114.923) (width 0.25) (layer "F.Cu") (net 7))
 (segment (start 135.923 114.923) (end 135.923 97.327) (width 0.25) (layer "F.Cu") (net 7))
 (segment (start 135.923 97.327) (end 138.5 94.75) (width 0.25) (layer "F.Cu") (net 7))
 (segment (start 138.8316 114.95) (end 138.8316 115.8316) (width 0.25) (layer "F.Cu") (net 6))
 (segment (start 138.8316 115.8316) (end 140.5 117.5) (width 0.25) (layer "F.Cu") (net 6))
 (segment (start 143 64) (end 141 66) (width 1) (layer "F.Cu") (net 1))
 (segment (start 138.7 80.7) (end 140.7 80.7) (width 0.5) (layer "F.Cu") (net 1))
 (segment (start 141 81) (end 141 66) (width 2) (layer "F.Cu") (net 1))
 (segment (start 140.7 65.7) (end 141 66) (width 0.25) (layer "F.Cu") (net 1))
 (segment (start 138.8316 112.1684) (end 139.5 111.5) (width 0.25) (layer "F.Cu") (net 1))
 (segment (start 138.8316 105.55) (end 138.8316 104.6684) (width 0.25) (layer "F.Cu") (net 1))
 (segment (start 145.725 64) (end 143 64) (width 1) (layer "F.Cu") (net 1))
 (segment (start 140.7 80.7) (end 141 81) (width 0.5) (layer "F.Cu") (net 1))
 (segment (start 138.75 91.25) (end 141 89) (width 2) (layer "F.Cu") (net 1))
 (segment (start 138.8316 104.6684) (end 140 103.5) (width 0.25) (layer "F.Cu") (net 1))
 (segment (start 138.8316 113.05) (end 138.8316 112.1684) (width 0.25) (layer "F.Cu") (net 1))
 (segment (start 138.7 65.7) (end 140.7 65.7) (width 0.25) (layer "F.Cu") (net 1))
 (segment (start 138.5 91.25) (end 138.75 91.25) (width 2) (layer "F.Cu") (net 1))
 (segment (start 141 89) (end 141 81) (width 2) (layer "F.Cu") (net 1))
 (via (at 139.5 111.5) (size 0.6) (drill 0.3) (layers "F.Cu" "B.Cu") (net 1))
 (via (at 140 103.5) (size 0.6) (drill 0.3) (layers "F.Cu" "B.Cu") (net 1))
 (segment (start 140 92.75) (end 138.5 91.25) (width 0.25) (layer "B.Cu") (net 1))
 (segment (start 140 103.5) (end 140 92.75) (width 0.25) (layer "B.Cu") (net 1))
 (segment (start 139.5 111.5) (end 140 111) (width 0.25) (layer "B.Cu") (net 1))
 (segment (start 140 111) (end 140 103.5) (width 0.25) (layer "B.Cu") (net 1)))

